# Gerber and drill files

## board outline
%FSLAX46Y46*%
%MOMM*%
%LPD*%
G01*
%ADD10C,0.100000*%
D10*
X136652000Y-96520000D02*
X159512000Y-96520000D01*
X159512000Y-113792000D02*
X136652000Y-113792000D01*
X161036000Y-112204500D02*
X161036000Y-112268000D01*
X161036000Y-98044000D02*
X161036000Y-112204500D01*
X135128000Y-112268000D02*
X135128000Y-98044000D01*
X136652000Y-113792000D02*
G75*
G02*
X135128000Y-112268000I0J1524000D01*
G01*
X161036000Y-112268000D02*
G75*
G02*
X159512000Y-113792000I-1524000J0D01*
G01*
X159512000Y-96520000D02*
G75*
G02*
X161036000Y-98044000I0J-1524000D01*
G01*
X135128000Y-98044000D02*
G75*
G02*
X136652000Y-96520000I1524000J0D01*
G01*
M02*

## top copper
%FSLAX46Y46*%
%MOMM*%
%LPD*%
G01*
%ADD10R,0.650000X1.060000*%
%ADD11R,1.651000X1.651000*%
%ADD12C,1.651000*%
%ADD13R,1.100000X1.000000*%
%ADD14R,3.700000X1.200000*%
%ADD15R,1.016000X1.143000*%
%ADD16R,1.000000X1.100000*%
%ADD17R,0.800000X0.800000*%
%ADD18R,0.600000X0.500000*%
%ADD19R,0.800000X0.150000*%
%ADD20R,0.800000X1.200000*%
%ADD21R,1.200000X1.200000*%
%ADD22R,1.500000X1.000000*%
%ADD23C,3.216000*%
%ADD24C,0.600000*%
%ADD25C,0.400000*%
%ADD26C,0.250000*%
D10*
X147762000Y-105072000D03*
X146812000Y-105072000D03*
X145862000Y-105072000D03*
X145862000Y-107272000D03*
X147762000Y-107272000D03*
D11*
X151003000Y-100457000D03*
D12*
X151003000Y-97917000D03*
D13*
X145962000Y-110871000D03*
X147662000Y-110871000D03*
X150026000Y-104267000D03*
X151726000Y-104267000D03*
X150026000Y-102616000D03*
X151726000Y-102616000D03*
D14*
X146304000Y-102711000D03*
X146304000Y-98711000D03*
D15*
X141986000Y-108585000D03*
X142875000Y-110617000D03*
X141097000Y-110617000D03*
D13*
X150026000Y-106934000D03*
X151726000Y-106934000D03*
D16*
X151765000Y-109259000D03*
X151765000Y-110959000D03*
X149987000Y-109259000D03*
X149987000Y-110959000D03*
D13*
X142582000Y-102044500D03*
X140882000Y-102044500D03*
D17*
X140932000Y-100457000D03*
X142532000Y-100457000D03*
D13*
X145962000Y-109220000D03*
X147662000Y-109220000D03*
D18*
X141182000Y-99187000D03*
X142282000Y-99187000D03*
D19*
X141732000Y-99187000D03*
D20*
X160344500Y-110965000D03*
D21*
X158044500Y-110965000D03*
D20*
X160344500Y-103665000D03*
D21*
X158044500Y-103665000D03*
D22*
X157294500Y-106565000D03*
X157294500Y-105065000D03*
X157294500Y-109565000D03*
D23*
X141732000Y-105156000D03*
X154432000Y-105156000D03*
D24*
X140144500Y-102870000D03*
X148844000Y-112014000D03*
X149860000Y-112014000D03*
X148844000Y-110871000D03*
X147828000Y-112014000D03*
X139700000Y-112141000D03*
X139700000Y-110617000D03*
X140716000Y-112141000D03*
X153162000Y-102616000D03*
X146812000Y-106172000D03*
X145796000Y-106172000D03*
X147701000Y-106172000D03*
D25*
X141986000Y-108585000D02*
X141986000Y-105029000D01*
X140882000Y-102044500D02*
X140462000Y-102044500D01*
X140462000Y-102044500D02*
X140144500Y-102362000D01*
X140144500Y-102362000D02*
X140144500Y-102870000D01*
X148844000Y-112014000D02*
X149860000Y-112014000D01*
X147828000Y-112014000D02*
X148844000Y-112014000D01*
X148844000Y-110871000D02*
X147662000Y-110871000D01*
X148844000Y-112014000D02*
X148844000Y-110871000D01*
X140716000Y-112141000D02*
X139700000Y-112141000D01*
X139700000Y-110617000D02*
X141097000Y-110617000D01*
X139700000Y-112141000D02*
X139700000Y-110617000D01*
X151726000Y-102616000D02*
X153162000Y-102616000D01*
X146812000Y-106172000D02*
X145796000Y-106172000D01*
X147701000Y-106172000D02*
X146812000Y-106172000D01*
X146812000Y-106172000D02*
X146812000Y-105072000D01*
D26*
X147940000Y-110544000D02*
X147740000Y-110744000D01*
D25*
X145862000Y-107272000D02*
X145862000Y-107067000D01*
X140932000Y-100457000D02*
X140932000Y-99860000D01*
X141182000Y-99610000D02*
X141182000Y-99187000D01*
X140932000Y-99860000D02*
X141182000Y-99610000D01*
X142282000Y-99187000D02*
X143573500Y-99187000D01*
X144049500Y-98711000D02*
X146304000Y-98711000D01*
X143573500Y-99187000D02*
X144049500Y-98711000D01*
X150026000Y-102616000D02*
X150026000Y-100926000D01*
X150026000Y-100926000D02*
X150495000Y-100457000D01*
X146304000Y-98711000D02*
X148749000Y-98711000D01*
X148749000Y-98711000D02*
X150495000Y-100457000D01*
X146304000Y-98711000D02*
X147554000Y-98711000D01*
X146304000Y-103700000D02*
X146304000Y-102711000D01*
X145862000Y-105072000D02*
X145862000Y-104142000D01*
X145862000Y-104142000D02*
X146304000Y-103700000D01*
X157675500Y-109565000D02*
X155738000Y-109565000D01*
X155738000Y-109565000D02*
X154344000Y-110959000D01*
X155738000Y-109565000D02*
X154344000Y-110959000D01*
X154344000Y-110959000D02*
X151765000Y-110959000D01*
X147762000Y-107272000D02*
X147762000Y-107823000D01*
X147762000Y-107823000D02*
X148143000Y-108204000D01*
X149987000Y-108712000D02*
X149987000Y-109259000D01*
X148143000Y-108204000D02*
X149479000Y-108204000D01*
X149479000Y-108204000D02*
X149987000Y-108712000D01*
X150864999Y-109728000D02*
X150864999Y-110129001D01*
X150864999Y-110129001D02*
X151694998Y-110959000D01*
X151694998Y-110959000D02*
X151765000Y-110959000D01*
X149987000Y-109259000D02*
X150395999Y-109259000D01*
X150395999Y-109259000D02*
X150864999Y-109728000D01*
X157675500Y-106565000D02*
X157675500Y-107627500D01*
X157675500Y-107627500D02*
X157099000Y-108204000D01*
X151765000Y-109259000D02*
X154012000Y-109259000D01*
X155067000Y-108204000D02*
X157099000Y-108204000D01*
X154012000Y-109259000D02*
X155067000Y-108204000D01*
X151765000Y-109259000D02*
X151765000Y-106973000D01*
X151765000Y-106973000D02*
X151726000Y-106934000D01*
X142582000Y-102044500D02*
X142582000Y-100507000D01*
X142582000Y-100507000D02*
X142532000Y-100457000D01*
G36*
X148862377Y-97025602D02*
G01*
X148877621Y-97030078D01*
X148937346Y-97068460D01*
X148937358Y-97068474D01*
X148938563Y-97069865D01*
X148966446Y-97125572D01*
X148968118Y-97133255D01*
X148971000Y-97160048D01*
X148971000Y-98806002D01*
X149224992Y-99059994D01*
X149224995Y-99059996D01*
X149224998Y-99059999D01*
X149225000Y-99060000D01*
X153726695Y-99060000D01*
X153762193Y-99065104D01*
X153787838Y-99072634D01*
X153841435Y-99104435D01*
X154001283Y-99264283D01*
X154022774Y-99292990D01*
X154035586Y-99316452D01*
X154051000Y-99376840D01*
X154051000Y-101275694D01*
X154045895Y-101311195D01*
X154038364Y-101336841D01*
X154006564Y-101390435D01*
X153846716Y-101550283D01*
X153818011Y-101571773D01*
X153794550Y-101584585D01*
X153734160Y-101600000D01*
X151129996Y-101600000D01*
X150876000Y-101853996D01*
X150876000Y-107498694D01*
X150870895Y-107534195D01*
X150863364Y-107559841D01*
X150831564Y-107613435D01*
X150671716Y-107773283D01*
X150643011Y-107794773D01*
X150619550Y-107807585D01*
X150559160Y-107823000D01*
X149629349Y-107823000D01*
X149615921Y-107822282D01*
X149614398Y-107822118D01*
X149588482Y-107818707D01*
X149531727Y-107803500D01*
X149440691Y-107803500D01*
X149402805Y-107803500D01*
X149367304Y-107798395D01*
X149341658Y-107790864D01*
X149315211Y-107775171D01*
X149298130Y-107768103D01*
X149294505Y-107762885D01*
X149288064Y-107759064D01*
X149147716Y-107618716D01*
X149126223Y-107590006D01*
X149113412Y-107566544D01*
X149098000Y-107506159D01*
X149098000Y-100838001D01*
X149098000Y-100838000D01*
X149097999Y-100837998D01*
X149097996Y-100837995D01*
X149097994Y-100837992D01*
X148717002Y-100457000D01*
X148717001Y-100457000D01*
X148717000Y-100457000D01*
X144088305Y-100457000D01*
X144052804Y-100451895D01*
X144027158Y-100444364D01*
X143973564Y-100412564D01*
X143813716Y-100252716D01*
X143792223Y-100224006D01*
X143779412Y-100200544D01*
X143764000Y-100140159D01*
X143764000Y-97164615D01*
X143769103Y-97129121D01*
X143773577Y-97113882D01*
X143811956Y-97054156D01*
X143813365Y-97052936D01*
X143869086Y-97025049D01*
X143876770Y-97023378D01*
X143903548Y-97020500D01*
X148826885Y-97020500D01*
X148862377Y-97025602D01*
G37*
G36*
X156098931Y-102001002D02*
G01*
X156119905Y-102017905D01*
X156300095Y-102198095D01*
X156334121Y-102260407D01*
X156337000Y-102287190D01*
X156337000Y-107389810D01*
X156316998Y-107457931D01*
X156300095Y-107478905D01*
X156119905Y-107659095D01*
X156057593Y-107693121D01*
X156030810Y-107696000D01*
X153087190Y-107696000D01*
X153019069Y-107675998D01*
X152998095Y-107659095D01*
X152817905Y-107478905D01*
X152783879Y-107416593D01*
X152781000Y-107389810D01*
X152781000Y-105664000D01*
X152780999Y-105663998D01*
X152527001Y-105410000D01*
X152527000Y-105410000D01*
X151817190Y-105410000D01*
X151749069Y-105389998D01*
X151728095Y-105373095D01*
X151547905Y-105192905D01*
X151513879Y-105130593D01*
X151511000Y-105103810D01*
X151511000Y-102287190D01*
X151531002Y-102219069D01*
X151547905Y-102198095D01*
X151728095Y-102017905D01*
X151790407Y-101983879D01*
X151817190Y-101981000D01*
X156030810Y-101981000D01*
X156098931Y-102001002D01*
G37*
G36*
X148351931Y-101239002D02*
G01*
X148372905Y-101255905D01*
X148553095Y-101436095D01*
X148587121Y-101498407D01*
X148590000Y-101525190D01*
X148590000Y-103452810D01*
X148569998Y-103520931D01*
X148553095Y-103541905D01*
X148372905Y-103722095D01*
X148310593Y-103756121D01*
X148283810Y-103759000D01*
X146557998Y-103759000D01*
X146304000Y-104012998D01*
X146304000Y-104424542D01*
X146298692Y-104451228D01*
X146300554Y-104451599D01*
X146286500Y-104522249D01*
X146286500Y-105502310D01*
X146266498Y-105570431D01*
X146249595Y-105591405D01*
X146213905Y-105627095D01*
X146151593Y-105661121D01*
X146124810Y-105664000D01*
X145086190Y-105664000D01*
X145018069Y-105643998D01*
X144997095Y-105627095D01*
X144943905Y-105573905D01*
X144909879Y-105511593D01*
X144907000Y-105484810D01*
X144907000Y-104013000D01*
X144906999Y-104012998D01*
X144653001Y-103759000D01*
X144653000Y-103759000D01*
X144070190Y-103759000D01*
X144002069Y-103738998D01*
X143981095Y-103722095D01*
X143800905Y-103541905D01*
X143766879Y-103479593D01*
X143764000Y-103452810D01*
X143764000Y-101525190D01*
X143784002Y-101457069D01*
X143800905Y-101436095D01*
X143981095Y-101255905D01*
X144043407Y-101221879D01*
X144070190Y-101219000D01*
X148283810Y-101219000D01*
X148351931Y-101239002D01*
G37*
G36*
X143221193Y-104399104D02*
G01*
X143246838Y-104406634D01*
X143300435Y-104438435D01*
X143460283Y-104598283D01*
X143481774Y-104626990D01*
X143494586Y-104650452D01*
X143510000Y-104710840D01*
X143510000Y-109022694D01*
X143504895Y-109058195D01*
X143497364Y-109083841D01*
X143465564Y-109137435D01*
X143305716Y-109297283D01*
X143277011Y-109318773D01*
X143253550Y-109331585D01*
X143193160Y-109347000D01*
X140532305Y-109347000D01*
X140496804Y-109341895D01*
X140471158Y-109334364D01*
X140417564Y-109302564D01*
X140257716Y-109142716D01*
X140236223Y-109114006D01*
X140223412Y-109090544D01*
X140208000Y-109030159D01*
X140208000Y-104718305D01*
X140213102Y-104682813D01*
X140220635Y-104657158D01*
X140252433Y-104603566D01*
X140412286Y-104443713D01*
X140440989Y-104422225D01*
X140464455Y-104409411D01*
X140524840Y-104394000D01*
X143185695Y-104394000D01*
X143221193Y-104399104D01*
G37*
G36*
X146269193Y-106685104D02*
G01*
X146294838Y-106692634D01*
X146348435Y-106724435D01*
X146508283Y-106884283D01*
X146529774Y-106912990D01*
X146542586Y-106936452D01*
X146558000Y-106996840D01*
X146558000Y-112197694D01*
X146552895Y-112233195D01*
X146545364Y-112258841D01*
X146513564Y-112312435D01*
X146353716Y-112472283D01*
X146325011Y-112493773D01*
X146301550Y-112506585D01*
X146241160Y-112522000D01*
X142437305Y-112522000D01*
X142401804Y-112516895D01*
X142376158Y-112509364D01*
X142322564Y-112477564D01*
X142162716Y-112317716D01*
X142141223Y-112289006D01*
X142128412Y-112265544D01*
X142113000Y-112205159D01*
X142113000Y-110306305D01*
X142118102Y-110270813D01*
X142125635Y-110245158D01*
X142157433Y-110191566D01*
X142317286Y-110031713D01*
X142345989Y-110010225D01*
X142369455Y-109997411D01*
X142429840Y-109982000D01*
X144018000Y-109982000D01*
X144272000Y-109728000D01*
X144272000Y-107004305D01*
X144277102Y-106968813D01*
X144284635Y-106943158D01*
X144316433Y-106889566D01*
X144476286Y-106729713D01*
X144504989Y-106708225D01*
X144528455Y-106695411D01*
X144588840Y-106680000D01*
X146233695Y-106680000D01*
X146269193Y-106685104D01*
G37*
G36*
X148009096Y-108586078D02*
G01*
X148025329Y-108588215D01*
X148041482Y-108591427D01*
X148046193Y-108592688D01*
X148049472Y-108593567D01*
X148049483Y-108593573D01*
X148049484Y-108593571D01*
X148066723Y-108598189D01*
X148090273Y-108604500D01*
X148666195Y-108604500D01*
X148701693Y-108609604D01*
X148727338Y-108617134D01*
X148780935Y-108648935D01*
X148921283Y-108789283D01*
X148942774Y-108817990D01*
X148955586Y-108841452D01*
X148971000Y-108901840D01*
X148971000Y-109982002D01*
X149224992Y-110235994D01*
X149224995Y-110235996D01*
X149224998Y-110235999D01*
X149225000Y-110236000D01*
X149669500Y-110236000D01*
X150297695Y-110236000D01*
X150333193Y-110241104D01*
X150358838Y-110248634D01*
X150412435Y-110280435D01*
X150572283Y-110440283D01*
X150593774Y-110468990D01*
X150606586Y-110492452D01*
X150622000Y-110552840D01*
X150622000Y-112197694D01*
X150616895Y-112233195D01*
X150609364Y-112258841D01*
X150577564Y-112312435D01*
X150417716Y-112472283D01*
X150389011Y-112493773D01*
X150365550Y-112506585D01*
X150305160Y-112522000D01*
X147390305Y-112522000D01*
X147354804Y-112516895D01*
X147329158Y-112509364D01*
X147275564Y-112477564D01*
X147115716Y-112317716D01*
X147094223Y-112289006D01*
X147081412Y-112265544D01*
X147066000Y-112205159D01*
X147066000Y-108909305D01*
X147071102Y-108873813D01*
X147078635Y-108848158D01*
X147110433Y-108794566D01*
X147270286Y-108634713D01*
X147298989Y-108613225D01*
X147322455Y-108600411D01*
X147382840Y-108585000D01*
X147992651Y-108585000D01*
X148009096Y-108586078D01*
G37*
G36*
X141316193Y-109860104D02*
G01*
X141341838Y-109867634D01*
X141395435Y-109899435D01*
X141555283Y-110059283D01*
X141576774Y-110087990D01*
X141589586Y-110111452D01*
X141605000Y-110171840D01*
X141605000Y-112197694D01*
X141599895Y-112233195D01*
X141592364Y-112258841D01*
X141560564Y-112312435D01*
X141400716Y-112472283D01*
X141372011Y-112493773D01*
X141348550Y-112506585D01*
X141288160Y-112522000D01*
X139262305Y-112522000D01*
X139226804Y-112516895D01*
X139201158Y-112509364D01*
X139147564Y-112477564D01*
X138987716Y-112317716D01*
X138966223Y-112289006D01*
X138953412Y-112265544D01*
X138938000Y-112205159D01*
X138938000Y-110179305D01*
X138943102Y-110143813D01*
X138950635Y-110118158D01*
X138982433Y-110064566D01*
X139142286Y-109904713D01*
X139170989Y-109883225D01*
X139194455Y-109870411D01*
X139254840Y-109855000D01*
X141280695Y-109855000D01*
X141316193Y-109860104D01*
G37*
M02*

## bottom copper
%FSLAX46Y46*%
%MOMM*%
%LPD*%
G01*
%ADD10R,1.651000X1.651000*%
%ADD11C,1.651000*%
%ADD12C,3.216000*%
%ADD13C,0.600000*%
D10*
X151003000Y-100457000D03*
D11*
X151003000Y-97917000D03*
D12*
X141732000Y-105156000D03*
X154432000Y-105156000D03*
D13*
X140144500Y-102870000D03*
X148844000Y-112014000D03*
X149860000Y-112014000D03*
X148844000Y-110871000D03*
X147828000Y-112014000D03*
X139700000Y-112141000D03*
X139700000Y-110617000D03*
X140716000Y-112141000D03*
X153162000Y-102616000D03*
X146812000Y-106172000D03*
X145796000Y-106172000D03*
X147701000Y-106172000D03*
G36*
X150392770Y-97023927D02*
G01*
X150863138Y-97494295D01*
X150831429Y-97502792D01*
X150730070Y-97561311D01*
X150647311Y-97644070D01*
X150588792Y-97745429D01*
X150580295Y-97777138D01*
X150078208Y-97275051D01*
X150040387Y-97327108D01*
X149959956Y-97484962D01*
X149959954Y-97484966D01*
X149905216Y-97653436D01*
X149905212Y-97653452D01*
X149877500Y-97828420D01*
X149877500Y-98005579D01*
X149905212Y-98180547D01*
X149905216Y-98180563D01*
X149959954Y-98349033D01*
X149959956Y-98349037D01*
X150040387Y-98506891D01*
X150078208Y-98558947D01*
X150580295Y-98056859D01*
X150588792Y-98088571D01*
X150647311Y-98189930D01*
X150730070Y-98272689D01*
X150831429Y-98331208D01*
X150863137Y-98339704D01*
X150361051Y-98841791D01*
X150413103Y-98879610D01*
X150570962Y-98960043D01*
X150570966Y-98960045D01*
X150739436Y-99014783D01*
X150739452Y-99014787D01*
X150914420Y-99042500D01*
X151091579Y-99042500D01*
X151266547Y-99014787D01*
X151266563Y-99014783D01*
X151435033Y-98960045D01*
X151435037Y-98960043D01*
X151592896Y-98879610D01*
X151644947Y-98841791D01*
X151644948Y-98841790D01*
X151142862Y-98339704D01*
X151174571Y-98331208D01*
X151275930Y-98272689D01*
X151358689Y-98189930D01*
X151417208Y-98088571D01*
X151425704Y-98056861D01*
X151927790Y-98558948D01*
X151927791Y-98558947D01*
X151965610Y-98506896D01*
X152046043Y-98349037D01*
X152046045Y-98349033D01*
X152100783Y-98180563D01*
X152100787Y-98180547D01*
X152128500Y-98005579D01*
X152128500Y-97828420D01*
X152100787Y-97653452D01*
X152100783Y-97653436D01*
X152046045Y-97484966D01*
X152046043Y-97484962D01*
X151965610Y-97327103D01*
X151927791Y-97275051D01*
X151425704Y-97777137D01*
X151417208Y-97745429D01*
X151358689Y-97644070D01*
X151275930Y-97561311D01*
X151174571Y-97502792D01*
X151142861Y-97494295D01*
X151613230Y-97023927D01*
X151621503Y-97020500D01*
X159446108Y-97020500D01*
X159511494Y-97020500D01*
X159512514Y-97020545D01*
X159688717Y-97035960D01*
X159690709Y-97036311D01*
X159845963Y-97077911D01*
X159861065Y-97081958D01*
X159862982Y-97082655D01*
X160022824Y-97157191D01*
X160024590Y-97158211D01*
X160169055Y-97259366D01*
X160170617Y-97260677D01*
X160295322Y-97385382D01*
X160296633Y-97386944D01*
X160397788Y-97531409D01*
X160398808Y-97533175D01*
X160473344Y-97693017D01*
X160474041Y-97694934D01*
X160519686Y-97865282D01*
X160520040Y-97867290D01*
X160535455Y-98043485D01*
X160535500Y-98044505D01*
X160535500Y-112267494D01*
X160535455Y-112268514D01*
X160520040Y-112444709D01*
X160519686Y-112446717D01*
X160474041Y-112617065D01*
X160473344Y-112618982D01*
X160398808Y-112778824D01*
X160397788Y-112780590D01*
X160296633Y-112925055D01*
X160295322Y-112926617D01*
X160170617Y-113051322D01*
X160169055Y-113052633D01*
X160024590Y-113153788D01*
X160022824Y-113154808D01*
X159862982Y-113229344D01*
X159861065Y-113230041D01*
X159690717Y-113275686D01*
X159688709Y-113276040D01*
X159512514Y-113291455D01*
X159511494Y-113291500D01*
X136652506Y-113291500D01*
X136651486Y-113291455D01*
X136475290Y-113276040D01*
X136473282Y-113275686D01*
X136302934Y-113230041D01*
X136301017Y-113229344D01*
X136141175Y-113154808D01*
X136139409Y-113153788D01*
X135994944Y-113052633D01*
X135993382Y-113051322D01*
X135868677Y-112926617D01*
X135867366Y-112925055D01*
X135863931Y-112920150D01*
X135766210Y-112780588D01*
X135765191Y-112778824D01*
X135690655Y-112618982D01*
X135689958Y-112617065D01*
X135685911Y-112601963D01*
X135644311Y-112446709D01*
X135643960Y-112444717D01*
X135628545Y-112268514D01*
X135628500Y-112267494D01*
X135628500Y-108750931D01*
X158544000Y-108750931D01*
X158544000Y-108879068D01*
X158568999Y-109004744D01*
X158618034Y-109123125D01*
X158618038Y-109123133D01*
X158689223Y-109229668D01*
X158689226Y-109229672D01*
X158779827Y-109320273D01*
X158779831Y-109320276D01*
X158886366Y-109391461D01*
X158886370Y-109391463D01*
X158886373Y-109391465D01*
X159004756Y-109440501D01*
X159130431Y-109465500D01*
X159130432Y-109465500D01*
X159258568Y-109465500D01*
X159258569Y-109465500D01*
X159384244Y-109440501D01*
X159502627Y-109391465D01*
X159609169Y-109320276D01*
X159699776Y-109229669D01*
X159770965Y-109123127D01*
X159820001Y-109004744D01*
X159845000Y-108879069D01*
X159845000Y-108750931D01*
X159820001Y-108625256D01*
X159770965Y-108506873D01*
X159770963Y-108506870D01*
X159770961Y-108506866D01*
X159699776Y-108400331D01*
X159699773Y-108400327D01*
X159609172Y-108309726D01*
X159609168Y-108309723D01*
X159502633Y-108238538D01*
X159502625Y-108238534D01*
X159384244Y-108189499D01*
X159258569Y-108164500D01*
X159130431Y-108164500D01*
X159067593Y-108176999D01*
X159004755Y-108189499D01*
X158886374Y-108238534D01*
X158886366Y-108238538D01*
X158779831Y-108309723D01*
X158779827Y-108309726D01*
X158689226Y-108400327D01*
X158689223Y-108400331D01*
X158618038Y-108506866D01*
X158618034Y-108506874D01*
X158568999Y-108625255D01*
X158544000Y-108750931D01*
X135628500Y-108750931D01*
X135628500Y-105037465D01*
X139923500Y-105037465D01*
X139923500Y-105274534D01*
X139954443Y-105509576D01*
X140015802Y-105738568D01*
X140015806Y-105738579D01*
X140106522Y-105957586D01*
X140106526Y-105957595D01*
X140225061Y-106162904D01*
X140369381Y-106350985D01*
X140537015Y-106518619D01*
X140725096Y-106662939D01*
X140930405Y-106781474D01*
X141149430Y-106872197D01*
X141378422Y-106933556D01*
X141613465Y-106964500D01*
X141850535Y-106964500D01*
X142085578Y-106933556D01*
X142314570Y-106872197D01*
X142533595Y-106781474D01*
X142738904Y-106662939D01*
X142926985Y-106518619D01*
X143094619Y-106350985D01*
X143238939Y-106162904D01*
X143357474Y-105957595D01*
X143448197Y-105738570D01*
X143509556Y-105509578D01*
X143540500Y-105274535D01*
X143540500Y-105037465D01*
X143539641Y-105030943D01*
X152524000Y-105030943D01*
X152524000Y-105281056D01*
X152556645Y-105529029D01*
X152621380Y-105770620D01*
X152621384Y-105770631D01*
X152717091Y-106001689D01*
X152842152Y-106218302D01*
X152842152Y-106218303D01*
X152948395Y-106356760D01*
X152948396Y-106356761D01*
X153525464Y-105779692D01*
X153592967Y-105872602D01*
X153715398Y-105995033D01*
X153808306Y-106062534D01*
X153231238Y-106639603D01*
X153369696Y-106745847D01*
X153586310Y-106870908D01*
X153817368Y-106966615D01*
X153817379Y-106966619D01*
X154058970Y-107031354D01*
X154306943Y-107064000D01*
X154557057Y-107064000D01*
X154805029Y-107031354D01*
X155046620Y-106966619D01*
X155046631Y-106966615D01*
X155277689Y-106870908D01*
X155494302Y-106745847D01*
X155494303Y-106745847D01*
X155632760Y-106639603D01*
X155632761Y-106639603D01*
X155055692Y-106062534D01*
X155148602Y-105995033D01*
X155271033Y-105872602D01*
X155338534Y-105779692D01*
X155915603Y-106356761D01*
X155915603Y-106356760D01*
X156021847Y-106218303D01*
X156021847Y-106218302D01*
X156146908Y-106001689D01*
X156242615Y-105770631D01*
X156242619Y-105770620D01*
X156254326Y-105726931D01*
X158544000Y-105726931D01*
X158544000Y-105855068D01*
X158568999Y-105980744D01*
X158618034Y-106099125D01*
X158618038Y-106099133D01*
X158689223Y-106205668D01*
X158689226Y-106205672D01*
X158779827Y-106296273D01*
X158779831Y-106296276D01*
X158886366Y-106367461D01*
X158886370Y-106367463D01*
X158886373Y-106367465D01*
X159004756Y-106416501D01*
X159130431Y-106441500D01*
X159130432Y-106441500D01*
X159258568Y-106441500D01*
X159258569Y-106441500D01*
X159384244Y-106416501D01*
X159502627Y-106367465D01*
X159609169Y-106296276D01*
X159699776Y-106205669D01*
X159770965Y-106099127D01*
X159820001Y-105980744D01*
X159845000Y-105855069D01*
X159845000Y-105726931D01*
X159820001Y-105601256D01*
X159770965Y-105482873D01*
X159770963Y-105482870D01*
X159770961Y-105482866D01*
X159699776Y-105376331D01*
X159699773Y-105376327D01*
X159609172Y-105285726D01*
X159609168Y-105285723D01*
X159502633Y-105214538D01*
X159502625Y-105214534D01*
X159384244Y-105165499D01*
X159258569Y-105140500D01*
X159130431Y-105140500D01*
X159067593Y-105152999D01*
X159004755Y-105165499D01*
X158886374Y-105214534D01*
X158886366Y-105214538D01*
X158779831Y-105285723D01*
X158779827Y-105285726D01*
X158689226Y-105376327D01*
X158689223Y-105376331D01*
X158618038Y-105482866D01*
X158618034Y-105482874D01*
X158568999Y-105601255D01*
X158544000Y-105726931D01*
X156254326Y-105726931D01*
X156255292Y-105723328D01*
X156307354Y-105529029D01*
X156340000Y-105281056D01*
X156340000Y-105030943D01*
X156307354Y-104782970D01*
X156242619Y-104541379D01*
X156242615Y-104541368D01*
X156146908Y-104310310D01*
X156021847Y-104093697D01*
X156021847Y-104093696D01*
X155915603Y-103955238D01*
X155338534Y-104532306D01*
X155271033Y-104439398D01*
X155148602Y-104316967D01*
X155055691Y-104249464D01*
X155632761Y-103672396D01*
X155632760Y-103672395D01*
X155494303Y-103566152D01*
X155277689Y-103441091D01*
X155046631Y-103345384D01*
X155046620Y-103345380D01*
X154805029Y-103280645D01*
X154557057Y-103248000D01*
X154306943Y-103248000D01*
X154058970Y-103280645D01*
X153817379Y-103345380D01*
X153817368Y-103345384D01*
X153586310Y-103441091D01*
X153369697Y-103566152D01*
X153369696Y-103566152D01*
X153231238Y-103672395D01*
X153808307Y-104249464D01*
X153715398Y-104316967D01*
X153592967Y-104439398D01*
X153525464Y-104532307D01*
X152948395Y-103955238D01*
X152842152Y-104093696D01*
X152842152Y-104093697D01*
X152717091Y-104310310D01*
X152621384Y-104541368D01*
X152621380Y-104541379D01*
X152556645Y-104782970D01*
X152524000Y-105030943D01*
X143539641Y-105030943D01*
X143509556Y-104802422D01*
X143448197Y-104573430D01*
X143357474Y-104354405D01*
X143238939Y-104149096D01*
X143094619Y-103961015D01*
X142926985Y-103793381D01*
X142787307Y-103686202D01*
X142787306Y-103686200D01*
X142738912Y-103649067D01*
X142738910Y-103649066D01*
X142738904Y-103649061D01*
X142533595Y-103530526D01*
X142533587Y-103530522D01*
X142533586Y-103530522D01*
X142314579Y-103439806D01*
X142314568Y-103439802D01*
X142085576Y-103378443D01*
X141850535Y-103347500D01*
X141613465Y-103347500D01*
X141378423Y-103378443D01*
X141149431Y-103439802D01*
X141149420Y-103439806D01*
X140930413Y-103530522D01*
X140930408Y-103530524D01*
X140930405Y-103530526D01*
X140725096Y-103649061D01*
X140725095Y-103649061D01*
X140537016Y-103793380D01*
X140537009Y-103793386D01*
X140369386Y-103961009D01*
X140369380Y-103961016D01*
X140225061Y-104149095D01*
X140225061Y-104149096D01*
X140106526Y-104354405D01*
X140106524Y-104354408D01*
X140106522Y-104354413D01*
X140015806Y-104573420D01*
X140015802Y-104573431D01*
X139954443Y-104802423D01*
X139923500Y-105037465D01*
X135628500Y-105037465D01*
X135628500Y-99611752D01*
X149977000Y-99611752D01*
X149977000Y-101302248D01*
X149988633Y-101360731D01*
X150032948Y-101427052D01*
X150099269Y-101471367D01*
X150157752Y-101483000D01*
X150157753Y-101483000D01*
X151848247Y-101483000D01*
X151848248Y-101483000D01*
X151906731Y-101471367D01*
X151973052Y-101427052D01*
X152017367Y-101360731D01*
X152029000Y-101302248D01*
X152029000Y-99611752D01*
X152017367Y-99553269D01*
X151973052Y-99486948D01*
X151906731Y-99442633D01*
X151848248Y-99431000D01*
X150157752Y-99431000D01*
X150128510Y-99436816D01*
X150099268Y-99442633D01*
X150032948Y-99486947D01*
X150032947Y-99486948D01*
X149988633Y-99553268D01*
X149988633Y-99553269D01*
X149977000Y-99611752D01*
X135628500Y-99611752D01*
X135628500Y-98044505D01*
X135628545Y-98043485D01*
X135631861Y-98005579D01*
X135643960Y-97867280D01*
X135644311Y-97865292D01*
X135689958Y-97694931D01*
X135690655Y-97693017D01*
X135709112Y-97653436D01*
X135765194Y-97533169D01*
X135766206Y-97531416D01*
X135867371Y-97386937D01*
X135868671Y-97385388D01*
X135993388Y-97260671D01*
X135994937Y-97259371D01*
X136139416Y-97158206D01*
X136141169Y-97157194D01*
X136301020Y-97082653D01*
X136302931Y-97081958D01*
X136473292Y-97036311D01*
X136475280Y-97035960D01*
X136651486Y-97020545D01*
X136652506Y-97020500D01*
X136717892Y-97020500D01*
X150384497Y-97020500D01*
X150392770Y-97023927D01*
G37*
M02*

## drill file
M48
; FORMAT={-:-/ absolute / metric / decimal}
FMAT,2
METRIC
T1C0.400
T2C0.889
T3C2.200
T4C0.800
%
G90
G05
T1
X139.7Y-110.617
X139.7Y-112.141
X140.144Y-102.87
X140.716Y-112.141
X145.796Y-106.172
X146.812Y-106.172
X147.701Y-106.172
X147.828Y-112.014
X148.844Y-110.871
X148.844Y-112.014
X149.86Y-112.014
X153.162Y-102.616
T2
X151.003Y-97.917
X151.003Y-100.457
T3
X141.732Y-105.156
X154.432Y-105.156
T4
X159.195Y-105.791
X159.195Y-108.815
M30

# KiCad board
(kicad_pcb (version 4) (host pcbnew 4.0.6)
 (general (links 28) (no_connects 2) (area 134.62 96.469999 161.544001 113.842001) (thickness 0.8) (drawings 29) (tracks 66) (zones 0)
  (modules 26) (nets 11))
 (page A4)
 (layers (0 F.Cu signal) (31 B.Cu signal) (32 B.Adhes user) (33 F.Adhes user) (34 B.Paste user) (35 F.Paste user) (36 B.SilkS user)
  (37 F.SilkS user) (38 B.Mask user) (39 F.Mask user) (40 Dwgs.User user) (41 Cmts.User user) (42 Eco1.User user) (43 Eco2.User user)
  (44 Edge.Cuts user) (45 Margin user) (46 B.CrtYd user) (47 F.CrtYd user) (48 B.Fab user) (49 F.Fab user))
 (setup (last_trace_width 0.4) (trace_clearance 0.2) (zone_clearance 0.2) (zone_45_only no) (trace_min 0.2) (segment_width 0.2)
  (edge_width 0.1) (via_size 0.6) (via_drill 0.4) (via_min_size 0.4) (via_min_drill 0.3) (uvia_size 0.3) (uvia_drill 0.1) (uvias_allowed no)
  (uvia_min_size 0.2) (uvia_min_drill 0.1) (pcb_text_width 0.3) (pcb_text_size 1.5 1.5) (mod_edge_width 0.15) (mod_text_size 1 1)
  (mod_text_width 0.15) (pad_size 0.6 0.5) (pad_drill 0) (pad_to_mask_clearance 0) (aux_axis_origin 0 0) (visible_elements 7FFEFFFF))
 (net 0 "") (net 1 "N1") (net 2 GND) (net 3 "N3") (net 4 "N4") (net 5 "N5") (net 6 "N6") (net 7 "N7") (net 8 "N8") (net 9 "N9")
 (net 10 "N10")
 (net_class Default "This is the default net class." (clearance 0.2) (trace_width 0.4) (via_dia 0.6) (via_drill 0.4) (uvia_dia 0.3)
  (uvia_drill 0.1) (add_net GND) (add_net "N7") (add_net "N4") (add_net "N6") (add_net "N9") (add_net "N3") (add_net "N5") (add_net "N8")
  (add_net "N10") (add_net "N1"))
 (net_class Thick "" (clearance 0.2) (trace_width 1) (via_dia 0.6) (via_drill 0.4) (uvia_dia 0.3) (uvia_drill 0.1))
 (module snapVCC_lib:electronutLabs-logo (layer F.Cu) (at 137.414 105.283 90)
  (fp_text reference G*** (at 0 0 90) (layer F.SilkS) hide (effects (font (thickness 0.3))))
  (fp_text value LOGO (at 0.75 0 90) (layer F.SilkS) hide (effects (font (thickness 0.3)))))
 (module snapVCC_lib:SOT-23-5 (layer F.Cu) (at 146.812 106.172 270)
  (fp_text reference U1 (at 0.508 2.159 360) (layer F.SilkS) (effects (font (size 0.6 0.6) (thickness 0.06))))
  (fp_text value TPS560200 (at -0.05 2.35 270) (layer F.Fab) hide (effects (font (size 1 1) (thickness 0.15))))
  (pad 1 smd rect (at -1.1 -0.95 270) (size 1.06 0.65) (layers F.Cu F.Paste F.Mask) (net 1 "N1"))
  (pad 2 smd rect (at -1.1 0 270) (size 1.06 0.65) (layers F.Cu F.Paste F.Mask) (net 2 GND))
  (pad 3 smd rect (at -1.1 0.95 270) (size 1.06 0.65) (layers F.Cu F.Paste F.Mask) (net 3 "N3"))
  (pad 4 smd rect (at 1.1 0.95 270) (size 1.06 0.65) (layers F.Cu F.Paste F.Mask) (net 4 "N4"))
  (pad 5 smd rect (at 1.1 -0.95 270) (size 1.06 0.65) (layers F.Cu F.Paste F.Mask) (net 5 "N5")))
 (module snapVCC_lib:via (layer F.Cu) (at 151.638 112.014)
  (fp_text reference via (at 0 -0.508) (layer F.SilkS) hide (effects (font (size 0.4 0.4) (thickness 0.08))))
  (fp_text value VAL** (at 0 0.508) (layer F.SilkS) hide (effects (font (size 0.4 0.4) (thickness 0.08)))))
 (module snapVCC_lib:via (layer F.Cu) (at 150.622 112.014)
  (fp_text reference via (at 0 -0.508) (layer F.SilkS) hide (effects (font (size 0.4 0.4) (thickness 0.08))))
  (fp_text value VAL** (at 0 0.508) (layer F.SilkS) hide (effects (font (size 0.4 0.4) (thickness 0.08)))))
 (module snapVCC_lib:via (layer F.Cu) (at 140.335 111.506)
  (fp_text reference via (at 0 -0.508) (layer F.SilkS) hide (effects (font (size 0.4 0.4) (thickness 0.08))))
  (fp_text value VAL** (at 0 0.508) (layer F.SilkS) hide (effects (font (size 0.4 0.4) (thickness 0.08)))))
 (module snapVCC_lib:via (layer F.Cu) (at 149.606 112.014)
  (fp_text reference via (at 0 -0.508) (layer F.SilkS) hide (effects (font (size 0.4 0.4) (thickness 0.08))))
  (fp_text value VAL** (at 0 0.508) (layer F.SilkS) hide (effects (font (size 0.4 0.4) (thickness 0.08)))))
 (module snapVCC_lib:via (layer F.Cu) (at 149.86 106.426)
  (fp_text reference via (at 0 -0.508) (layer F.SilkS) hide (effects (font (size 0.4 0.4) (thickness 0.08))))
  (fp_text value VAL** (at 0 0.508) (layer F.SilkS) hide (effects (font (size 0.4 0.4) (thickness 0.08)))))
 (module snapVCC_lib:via (layer F.Cu) (at 147.828 106.426)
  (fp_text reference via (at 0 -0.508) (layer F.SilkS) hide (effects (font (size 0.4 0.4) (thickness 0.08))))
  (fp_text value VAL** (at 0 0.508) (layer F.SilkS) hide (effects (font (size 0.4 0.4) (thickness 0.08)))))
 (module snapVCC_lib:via (layer F.Cu) (at 148.844 106.426)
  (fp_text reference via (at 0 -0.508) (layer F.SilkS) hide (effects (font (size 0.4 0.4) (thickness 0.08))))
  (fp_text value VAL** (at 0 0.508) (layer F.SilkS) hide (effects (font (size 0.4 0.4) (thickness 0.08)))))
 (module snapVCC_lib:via (layer F.Cu) (at 139.573 101.6)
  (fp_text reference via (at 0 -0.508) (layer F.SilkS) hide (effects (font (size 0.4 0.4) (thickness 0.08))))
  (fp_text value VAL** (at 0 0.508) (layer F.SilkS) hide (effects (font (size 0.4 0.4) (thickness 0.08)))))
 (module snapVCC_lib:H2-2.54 (layer F.Cu) (at 151.003 99.187 180)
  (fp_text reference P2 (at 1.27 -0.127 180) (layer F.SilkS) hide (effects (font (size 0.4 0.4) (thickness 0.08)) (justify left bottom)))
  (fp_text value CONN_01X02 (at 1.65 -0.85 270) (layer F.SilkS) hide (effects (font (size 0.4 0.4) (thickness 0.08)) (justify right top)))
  (pad 1 thru_hole rect (at 0 -1.27 180) (size 1.651 1.651) (drill 0.889) (layers *.Cu *.Mask) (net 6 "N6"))
  (pad 2 thru_hole circle (at 0 1.27 180) (size 1.651 1.651) (drill 0.889) (layers *.Cu *.Mask) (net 2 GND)))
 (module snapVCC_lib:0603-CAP (layer F.Cu) (at 146.812 110.871)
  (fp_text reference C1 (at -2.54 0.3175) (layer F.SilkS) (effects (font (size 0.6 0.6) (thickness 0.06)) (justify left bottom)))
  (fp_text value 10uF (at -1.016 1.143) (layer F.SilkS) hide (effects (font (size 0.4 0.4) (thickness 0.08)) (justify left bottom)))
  (pad 1 smd rect (at -0.85 0) (size 1.1 1) (layers F.Cu F.Paste F.Mask) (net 4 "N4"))
  (pad 2 smd rect (at 0.85 0) (size 1.1 1) (layers F.Cu F.Paste F.Mask) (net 2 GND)))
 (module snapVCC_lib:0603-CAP (layer F.Cu) (at 150.876 104.267)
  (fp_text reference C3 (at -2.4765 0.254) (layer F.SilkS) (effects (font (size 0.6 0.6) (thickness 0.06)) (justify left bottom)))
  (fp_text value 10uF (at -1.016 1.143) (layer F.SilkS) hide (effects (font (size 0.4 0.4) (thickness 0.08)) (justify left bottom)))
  (pad 1 smd rect (at -0.85 0) (size 1.1 1) (layers F.Cu F.Paste F.Mask) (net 6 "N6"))
  (pad 2 smd rect (at 0.85 0) (size 1.1 1) (layers F.Cu F.Paste F.Mask) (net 2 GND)))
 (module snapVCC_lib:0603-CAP (layer F.Cu) (at 150.876 102.616)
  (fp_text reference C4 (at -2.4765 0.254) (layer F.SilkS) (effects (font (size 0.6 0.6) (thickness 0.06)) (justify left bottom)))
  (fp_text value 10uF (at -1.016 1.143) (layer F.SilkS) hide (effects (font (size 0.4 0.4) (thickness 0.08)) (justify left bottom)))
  (pad 1 smd rect (at -0.85 0) (size 1.1 1) (layers F.Cu F.Paste F.Mask) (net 6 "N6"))
  (pad 2 smd rect (at 0.85 0) (size 1.1 1) (layers F.Cu F.Paste F.Mask) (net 2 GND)))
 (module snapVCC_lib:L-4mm (layer F.Cu) (at 146.304 100.711 90)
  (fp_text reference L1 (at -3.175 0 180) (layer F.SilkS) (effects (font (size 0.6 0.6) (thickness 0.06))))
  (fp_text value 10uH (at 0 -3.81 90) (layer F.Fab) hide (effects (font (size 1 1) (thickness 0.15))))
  (pad 1 smd rect (at -2 0 90) (size 1.2 3.7) (layers F.Cu F.Paste F.Mask) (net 3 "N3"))
  (pad 2 smd rect (at 2 0 90) (size 1.2 3.7) (layers F.Cu F.Paste F.Mask) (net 6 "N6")))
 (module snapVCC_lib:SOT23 (layer F.Cu) (at 141.986 109.601)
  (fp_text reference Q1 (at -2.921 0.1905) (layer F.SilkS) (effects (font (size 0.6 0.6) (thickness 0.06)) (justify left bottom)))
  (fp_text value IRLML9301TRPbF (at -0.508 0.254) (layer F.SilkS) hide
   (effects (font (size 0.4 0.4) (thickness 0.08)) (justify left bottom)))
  (pad 3 smd rect (at 0 -1.016) (size 1.016 1.143) (layers F.Cu F.Paste F.Mask) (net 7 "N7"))
  (pad 2 smd rect (at 0.889 1.016) (size 1.016 1.143) (layers F.Cu F.Paste F.Mask) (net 4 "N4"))
  (pad 1 smd rect (at -0.889 1.016 180) (size 1.016 1.143) (layers F.Cu F.Paste F.Mask) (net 2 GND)))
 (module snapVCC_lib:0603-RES (layer F.Cu) (at 150.876 106.934)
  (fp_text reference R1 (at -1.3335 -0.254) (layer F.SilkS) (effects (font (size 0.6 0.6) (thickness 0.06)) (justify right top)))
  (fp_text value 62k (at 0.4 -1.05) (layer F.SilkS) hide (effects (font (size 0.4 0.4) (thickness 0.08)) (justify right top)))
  (pad 1 smd rect (at -0.85 0) (size 1.1 1) (layers F.Cu F.Paste F.Mask) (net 6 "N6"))
  (pad 2 smd rect (at 0.85 0) (size 1.1 1) (layers F.Cu F.Paste F.Mask) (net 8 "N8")))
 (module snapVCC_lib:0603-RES (layer F.Cu) (at 151.765 110.109 270)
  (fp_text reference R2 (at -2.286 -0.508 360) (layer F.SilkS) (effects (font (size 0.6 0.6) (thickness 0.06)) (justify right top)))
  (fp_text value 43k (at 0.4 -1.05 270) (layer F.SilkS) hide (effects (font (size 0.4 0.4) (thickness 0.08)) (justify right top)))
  (pad 1 smd rect (at -0.85 0 270) (size 1.1 1) (layers F.Cu F.Paste F.Mask) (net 8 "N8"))
  (pad 2 smd rect (at 0.85 0 270) (size 1.1 1) (layers F.Cu F.Paste F.Mask) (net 5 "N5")))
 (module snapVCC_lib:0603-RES (layer F.Cu) (at 149.987 110.109 270)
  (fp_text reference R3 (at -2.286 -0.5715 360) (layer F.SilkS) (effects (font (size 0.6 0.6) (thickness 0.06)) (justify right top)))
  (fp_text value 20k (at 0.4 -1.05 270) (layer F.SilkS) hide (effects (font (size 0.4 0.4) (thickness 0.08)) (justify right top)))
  (pad 1 smd rect (at -0.85 0 270) (size 1.1 1) (layers F.Cu F.Paste F.Mask) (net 5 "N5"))
  (pad 2 smd rect (at 0.85 0 270) (size 1.1 1) (layers F.Cu F.Paste F.Mask) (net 2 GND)))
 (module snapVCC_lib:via (layer F.Cu) (at 140.335 110.49)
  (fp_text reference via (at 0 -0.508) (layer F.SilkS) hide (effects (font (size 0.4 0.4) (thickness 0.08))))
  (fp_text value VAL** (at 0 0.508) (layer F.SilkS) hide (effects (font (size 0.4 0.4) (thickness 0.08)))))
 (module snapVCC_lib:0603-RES (layer F.Cu) (at 141.732 102.0445 180)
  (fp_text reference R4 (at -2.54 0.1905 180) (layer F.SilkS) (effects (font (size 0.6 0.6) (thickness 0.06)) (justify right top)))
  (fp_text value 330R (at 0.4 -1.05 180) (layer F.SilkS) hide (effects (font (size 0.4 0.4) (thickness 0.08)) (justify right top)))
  (pad 1 smd rect (at -0.85 0 180) (size 1.1 1) (layers F.Cu F.Paste F.Mask) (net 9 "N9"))
  (pad 2 smd rect (at 0.85 0 180) (size 1.1 1) (layers F.Cu F.Paste F.Mask) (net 2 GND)))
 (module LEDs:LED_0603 (layer F.Cu) (at 141.732 100.457 180)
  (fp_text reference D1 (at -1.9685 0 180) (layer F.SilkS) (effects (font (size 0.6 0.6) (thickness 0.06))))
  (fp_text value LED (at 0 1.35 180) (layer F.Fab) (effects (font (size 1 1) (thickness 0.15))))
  (pad 2 smd rect (at 0.8 0) (size 0.8 0.8) (layers F.Cu F.Paste F.Mask) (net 6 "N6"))
  (pad 1 smd rect (at -0.8 0) (size 0.8 0.8) (layers F.Cu F.Paste F.Mask) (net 9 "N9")))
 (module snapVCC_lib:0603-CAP (layer F.Cu) (at 146.812 109.22)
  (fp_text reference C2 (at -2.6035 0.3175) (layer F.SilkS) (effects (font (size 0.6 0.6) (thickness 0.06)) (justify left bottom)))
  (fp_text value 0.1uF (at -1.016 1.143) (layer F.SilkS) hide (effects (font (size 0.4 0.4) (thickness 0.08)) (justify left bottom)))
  (pad 1 smd rect (at -0.85 0) (size 1.1 1) (layers F.Cu F.Paste F.Mask) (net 4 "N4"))
  (pad 2 smd rect (at 0.85 0) (size 1.1 1) (layers F.Cu F.Paste F.Mask) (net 2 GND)))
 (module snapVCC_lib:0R (layer F.Cu) (at 141.732 99.187)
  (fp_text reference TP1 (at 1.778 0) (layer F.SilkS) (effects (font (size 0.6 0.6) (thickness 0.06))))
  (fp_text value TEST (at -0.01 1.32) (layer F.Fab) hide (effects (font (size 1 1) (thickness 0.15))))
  (pad 1 smd rect (at -0.55 0) (size 0.6 0.5) (layers F.Cu F.Paste F.Mask) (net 6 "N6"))
  (pad 1 smd rect (at 0.55 0) (size 0.6 0.5) (layers F.Cu F.Paste F.Mask) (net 6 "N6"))
  (pad 1 smd rect (at 0 0) (size 0.8 0.15) (layers F.Cu F.Paste F.Mask) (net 6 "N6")))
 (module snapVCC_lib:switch (layer F.Cu) (at 159.1945 107.315 90)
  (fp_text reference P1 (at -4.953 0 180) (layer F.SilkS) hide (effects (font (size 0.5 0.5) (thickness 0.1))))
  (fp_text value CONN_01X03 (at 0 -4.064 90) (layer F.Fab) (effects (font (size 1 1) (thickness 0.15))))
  (pad "" np_thru_hole circle (at 1.524 0 90) (size 0.8 0.8) (drill 0.8) (layers *.Cu *.Mask F.SilkS))
  (pad "" np_thru_hole circle (at -1.5 0 90) (size 0.8 0.8) (drill 0.8) (layers *.Cu *.Mask F.SilkS))
  (pad "" smd rect (at -3.65 1.15 90) (size 1.2 0.8) (layers F.Cu F.Paste F.Mask))
  (pad "" smd rect (at -3.65 -1.15 90) (size 1.2 1.2) (layers F.Cu F.Paste F.Mask))
  (pad "" smd rect (at 3.65 1.15 90) (size 1.2 0.8) (layers F.Cu F.Paste F.Mask))
  (pad "" smd rect (at 3.65 -1.15 90) (size 1.2 1.2) (layers F.Cu F.Paste F.Mask))
  (pad 2 smd rect (at 0.75 -1.9 90) (size 1 1.5) (layers F.Cu F.Paste F.Mask) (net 8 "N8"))
  (pad 3 smd rect (at 2.25 -1.9 90) (size 1 1.5) (layers F.Cu F.Paste F.Mask) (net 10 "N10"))
  (pad 1 smd rect (at -2.25 -1.9 90) (size 1 1.5) (layers F.Cu F.Paste F.Mask) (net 5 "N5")))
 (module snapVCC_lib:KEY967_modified (layer B.Cu) (at 148.082 105.156)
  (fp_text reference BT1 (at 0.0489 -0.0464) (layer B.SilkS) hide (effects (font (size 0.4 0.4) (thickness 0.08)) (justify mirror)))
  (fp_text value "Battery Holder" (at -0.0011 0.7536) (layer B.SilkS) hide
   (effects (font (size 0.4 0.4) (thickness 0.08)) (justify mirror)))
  (pad 1 thru_hole circle (at -6.35 0) (size 3.216 3.216) (drill 2.2) (layers *.Cu *.Mask) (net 7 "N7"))
  (pad 2 thru_hole circle (at 6.35 0) (size 3.216 3.216) (drill 2.2) (layers *.Cu *.Mask) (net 2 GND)))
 (gr_line (start 136.652 96.52) (end 159.512 96.52) (angle 90) (layer Edge.Cuts) (width 0.1))
 (gr_line (start 159.512 113.792) (end 136.652 113.792) (angle 90) (layer Edge.Cuts) (width 0.1))
 (gr_line (start 161.036 112.2045) (end 161.036 112.268) (angle 90) (layer Edge.Cuts) (width 0.1))
 (gr_line (start 161.036 98.044) (end 161.036 112.2045) (angle 90) (layer Edge.Cuts) (width 0.1))
 (gr_line (start 135.128 112.268) (end 135.128 98.044) (angle 90) (layer Edge.Cuts) (width 0.1))
 (gr_arc (start 136.652 112.268) (end 136.652 113.792) (angle 90) (layer Edge.Cuts) (width 0.1))
 (gr_arc (start 159.512 112.268) (end 161.036 112.268) (angle 90) (layer Edge.Cuts) (width 0.1))
 (gr_arc (start 159.512 98.044) (end 159.512 96.52) (angle 90) (layer Edge.Cuts) (width 0.1))
 (gr_arc (start 136.652 98.044) (end 135.128 98.044) (angle 90) (layer Edge.Cuts) (width 0.1))
 (segment (start 141.986 108.585) (end 141.986 105.029) (width 0.4) (layer F.Cu) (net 7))
 (segment (start 140.882 102.0445) (end 140.462 102.0445) (width 0.4) (layer F.Cu) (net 2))
 (segment (start 140.462 102.0445) (end 140.1445 102.362) (width 0.4) (layer F.Cu) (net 2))
 (segment (start 140.1445 102.362) (end 140.1445 102.87) (width 0.4) (layer F.Cu) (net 2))
 (via (at 140.1445 102.87) (size 0.6) (drill 0.4) (layers F.Cu B.Cu) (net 2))
 (segment (start 148.844 112.014) (end 149.86 112.014) (width 0.4) (layer F.Cu) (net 2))
 (via (at 148.844 112.014) (size 0.6) (drill 0.4) (layers F.Cu B.Cu) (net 2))
 (via (at 149.86 112.014) (size 0.6) (drill 0.4) (layers F.Cu B.Cu) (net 2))
 (segment (start 147.828 112.014) (end 148.844 112.014) (width 0.4) (layer F.Cu) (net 2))
 (via (at 148.844 110.871) (size 0.6) (drill 0.4) (layers F.Cu B.Cu) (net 2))
 (segment (start 148.844 110.871) (end 147.662 110.871) (width 0.4) (layer F.Cu) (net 2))
 (segment (start 148.844 112.014) (end 148.844 110.871) (width 0.4) (layer F.Cu) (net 2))
 (via (at 147.828 112.014) (size 0.6) (drill 0.4) (layers F.Cu B.Cu) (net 2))
 (segment (start 140.716 112.141) (end 139.7 112.141) (width 0.4) (layer F.Cu) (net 2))
 (via (at 139.7 112.141) (size 0.6) (drill 0.4) (layers F.Cu B.Cu) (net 2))
 (segment (start 139.7 110.617) (end 141.097 110.617) (width 0.4) (layer F.Cu) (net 2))
 (via (at 139.7 110.617) (size 0.6) (drill 0.4) (layers F.Cu B.Cu) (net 2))
 (segment (start 139.7 112.141) (end 139.7 110.617) (width 0.4) (layer F.Cu) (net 2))
 (via (at 140.716 112.141) (size 0.6) (drill 0.4) (layers F.Cu B.Cu) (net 2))
 (segment (start 151.726 102.616) (end 153.162 102.616) (width 0.4) (layer F.Cu) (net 2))
 (via (at 153.162 102.616) (size 0.6) (drill 0.4) (layers F.Cu B.Cu) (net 2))
 (segment (start 146.812 106.172) (end 145.796 106.172) (width 0.4) (layer F.Cu) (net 2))
 (via (at 146.812 106.172) (size 0.6) (drill 0.4) (layers F.Cu B.Cu) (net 2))
 (via (at 145.796 106.172) (size 0.6) (drill 0.4) (layers F.Cu B.Cu) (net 2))
 (segment (start 147.701 106.172) (end 146.812 106.172) (width 0.4) (layer F.Cu) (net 2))
 (segment (start 146.812 106.172) (end 146.812 105.072) (width 0.4) (layer F.Cu) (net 2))
 (via (at 147.701 106.172) (size 0.6) (drill 0.4) (layers F.Cu B.Cu) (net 2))
 (segment (start 147.94 110.544) (end 147.74 110.744) (width 0.25) (layer F.Cu) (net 2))
 (segment (start 145.862 107.272) (end 145.862 107.067) (width 0.4) (layer F.Cu) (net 4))
 (segment (start 140.932 100.457) (end 140.932 99.86) (width 0.4) (layer F.Cu) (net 6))
 (segment (start 141.182 99.61) (end 141.182 99.187) (width 0.4) (layer F.Cu) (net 6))
 (segment (start 140.932 99.86) (end 141.182 99.61) (width 0.4) (layer F.Cu) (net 6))
 (segment (start 142.282 99.187) (end 143.5735 99.187) (width 0.4) (layer F.Cu) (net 6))
 (segment (start 144.0495 98.711) (end 146.304 98.711) (width 0.4) (layer F.Cu) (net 6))
 (segment (start 143.5735 99.187) (end 144.0495 98.711) (width 0.4) (layer F.Cu) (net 6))
 (segment (start 150.026 102.616) (end 150.026 100.926) (width 0.4) (layer F.Cu) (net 6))
 (segment (start 150.026 100.926) (end 150.495 100.457) (width 0.4) (layer F.Cu) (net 6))
 (segment (start 146.304 98.711) (end 148.749 98.711) (width 0.4) (layer F.Cu) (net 6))
 (segment (start 148.749 98.711) (end 150.495 100.457) (width 0.4) (layer F.Cu) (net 6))
 (segment (start 146.304 98.711) (end 147.554 98.711) (width 0.4) (layer F.Cu) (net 6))
 (segment (start 146.304 103.7) (end 146.304 102.711) (width 0.4) (layer F.Cu) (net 3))
 (segment (start 145.862 105.072) (end 145.862 104.142) (width 0.4) (layer F.Cu) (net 3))
 (segment (start 145.862 104.142) (end 146.304 103.7) (width 0.4) (layer F.Cu) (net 3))
 (segment (start 157.6755 109.565) (end 155.738 109.565) (width 0.4) (layer F.Cu) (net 5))
 (segment (start 155.738 109.565) (end 154.344 110.959) (width 0.4) (layer F.Cu) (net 5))
 (segment (start 155.738 109.565) (end 154.344 110.959) (width 0.4) (layer F.Cu) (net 5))
 (segment (start 154.344 110.959) (end 151.765 110.959) (width 0.4) (layer F.Cu) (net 5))
 (segment (start 147.762 107.272) (end 147.762 107.823) (width 0.4) (layer F.Cu) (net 5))
 (segment (start 147.762 107.823) (end 148.143 108.204) (width 0.4) (layer F.Cu) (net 5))
 (segment (start 149.987 108.712) (end 149.987 109.259) (width 0.4) (layer F.Cu) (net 5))
 (segment (start 148.143 108.204) (end 149.479 108.204) (width 0.4) (layer F.Cu) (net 5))
 (segment (start 149.479 108.204) (end 149.987 108.712) (width 0.4) (layer F.Cu) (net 5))
 (segment (start 150.864999 109.728) (end 150.864999 110.129001) (width 0.4) (layer F.Cu) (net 5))
 (segment (start 150.864999 110.129001) (end 151.694998 110.959) (width 0.4) (layer F.Cu) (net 5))
 (segment (start 151.694998 110.959) (end 151.765 110.959) (width 0.4) (layer F.Cu) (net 5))
 (segment (start 149.987 109.259) (end 150.395999 109.259) (width 0.4) (layer F.Cu) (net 5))
 (segment (start 150.395999 109.259) (end 150.864999 109.728) (width 0.4) (layer F.Cu) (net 5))
 (segment (start 157.6755 106.565) (end 157.6755 107.6275) (width 0.4) (layer F.Cu) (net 8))
 (segment (start 157.6755 107.6275) (end 157.099 108.204) (width 0.4) (layer F.Cu) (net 8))
 (segment (start 151.765 109.259) (end 154.012 109.259) (width 0.4) (layer F.Cu) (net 8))
 (segment (start 155.067 108.204) (end 157.099 108.204) (width 0.4) (layer F.Cu) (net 8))
 (segment (start 154.012 109.259) (end 155.067 108.204) (width 0.4) (layer F.Cu) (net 8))
 (segment (start 151.765 109.259) (end 151.765 106.973) (width 0.4) (layer F.Cu) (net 8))
 (segment (start 151.765 106.973) (end 151.726 106.934) (width 0.4) (layer F.Cu) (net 8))
 (segment (start 142.582 102.0445) (end 142.582 100.507) (width 0.4) (layer F.Cu) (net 9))
 (segment (start 142.582 100.507) (end 142.532 100.457) (width 0.4) (layer F.Cu) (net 9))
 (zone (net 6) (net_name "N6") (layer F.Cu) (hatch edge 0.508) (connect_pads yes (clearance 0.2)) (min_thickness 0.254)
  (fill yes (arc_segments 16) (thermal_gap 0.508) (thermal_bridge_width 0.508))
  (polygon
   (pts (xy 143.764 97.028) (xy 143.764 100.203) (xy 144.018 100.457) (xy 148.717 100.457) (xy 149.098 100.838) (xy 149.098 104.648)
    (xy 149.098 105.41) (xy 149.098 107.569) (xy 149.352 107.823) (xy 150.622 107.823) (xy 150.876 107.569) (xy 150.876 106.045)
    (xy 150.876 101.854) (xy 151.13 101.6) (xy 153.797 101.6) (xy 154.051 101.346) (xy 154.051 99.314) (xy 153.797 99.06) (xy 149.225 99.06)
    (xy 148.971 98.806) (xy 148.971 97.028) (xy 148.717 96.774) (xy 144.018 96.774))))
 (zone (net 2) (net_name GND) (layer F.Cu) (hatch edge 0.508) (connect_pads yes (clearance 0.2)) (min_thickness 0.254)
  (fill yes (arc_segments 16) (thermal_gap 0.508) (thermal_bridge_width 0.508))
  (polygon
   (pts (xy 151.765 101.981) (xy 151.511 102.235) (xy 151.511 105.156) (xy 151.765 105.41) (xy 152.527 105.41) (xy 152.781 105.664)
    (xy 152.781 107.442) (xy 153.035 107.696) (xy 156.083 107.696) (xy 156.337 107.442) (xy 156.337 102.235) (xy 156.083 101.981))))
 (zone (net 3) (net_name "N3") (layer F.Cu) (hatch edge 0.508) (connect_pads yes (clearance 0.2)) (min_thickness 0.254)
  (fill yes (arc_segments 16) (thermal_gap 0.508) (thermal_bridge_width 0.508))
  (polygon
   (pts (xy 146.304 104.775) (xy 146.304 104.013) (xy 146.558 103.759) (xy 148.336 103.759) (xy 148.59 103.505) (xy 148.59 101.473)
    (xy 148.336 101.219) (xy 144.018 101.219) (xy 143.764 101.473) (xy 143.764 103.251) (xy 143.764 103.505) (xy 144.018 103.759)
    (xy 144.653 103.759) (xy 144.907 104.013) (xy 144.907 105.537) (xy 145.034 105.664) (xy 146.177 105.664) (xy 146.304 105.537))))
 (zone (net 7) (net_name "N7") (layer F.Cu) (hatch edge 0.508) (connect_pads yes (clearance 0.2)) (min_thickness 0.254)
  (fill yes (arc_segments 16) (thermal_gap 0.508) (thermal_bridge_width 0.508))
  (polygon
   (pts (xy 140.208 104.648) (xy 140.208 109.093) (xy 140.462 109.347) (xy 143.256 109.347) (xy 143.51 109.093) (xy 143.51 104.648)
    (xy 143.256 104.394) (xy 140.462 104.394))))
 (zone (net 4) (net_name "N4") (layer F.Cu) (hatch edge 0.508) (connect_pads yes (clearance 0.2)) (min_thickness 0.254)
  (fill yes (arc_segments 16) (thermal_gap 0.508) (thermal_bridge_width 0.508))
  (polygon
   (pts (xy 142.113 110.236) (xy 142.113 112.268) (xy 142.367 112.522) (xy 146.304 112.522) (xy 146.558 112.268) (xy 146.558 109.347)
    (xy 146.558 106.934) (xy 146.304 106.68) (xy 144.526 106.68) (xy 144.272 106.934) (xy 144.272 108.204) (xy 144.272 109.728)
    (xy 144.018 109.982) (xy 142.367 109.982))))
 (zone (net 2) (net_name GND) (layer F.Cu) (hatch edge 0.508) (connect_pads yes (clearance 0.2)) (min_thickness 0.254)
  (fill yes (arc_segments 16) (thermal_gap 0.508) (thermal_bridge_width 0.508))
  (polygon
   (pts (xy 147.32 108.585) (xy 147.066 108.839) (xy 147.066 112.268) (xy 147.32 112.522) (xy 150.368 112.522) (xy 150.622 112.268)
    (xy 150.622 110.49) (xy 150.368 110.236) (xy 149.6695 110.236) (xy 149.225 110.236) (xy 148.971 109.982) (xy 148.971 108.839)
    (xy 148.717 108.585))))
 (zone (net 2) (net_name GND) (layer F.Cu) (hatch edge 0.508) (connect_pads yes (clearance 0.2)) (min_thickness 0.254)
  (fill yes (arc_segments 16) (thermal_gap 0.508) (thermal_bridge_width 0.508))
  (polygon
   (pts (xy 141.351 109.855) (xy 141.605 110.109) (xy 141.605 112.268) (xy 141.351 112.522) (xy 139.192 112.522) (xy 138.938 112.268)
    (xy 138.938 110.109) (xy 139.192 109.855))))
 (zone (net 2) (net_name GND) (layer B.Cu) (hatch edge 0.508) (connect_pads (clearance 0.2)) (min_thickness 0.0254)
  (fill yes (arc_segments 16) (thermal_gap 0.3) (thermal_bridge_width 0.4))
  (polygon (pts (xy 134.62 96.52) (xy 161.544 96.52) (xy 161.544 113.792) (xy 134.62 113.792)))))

